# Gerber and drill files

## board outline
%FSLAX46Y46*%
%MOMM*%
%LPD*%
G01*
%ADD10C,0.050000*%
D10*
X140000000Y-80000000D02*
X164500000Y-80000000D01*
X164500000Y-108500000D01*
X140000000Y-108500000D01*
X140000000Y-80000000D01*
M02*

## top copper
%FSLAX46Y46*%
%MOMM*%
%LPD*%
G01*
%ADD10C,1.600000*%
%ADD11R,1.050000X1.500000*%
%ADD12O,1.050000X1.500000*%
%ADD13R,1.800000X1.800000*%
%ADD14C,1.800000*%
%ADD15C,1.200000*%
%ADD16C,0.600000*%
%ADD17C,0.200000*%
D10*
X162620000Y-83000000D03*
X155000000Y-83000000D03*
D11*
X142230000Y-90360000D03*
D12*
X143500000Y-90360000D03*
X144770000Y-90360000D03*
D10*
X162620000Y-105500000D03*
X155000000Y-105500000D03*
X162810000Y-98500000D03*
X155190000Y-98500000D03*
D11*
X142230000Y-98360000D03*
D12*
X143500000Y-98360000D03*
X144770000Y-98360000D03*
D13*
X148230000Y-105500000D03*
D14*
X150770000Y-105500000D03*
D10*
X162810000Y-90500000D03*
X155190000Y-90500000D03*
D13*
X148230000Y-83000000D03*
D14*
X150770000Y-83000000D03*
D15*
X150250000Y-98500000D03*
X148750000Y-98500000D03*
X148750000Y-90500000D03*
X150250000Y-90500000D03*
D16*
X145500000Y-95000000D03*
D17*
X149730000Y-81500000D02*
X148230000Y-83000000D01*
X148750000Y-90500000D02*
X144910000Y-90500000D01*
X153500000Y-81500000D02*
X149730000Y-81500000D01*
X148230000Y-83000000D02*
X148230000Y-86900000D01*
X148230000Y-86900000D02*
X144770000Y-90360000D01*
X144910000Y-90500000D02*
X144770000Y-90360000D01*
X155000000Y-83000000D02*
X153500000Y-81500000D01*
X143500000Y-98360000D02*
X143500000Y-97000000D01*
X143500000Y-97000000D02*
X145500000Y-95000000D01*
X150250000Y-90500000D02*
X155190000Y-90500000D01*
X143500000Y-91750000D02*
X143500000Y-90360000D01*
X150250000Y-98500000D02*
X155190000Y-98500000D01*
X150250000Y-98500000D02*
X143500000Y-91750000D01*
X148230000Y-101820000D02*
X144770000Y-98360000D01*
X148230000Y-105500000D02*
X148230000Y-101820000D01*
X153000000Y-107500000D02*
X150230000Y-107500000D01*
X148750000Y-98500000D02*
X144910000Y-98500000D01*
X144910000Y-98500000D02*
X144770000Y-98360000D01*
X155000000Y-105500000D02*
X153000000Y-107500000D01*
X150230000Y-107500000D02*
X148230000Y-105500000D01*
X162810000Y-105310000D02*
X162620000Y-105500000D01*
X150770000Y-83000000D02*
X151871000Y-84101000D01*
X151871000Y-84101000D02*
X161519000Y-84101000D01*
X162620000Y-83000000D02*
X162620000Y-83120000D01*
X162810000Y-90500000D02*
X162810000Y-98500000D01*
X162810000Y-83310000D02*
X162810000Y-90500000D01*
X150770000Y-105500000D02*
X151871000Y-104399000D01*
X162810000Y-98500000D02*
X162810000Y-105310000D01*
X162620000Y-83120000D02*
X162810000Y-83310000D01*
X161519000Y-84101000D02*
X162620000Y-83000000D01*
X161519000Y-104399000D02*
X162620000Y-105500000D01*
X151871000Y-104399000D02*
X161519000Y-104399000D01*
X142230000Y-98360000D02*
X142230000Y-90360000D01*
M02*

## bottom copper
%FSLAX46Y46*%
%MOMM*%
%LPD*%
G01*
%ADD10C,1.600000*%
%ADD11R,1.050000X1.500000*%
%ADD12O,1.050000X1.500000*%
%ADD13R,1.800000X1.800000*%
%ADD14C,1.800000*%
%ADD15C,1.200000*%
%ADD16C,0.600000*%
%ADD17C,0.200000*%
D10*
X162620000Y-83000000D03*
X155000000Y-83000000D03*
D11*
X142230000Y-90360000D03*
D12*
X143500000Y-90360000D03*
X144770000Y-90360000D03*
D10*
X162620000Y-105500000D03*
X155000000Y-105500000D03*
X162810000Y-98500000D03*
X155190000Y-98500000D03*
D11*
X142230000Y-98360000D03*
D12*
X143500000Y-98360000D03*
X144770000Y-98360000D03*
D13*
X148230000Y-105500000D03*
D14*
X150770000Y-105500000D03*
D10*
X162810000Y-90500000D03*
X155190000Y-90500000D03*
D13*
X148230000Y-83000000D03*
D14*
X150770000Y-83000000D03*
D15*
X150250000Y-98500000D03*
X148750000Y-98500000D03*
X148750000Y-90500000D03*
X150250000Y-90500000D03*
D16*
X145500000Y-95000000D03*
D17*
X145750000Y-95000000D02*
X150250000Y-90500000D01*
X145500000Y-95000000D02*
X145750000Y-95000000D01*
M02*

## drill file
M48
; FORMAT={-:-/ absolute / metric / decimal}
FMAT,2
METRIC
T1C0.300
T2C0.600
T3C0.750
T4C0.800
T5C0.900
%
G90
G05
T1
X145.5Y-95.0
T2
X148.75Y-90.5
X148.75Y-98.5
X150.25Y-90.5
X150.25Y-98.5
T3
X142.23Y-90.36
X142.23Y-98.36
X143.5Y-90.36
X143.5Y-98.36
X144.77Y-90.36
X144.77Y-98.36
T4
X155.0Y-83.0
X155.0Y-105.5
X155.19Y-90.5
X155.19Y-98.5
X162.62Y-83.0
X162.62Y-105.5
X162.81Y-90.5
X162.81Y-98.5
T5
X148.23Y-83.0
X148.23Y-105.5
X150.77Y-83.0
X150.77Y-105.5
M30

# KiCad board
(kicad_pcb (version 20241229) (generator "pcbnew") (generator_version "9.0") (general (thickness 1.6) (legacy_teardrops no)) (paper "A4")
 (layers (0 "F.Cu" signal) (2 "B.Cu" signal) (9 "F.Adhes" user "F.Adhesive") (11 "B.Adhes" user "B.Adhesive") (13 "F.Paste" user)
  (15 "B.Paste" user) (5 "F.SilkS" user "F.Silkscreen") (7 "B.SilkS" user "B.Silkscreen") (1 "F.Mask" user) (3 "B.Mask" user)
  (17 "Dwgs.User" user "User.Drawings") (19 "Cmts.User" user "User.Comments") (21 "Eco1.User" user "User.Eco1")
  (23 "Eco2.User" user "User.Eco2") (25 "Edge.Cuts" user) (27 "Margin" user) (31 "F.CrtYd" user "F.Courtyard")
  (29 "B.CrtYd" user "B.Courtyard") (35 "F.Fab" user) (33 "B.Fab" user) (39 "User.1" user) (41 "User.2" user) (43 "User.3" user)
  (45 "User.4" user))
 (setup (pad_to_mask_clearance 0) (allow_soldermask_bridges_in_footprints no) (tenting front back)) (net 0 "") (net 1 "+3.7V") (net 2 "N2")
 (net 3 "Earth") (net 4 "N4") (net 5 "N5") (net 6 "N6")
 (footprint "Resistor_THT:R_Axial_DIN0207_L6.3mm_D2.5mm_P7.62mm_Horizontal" (layer "F.Cu") (at 162.62 83 180)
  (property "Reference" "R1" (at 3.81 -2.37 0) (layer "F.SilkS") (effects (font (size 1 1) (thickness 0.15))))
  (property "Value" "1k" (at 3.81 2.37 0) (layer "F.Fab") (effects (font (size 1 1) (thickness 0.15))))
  (pad "1" thru_hole circle (at 0 0 180) (size 1.6 1.6) (drill 0.8) (layers "*.Cu" "*.Mask") (remove_unused_layers no) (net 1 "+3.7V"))
  (pad "2" thru_hole circle (at 7.62 0 180) (size 1.6 1.6) (drill 0.8) (layers "*.Cu" "*.Mask") (remove_unused_layers no) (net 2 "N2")))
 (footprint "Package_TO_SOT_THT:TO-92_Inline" (layer "F.Cu") (at 142.23 90.36)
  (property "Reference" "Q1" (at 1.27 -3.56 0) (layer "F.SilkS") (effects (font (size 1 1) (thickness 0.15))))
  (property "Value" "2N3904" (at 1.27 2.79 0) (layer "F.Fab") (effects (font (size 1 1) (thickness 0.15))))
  (pad "1" thru_hole rect (at 0 0) (size 1.05 1.5) (drill 0.75) (layers "*.Cu" "*.Mask") (remove_unused_layers no) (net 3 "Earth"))
  (pad "2" thru_hole oval (at 1.27 0) (size 1.05 1.5) (drill 0.75) (layers "*.Cu" "*.Mask") (remove_unused_layers no) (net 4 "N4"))
  (pad "3" thru_hole oval (at 2.54 0) (size 1.05 1.5) (drill 0.75) (layers "*.Cu" "*.Mask") (remove_unused_layers no) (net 2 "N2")))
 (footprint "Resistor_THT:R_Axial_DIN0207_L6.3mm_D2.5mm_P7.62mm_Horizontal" (layer "F.Cu") (at 162.62 105.5 180)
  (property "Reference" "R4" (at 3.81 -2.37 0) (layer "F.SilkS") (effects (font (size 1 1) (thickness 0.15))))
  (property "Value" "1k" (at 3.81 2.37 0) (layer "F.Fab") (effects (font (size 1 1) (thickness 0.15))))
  (pad "1" thru_hole circle (at 0 0 180) (size 1.6 1.6) (drill 0.8) (layers "*.Cu" "*.Mask") (remove_unused_layers no) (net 1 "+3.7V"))
  (pad "2" thru_hole circle (at 7.62 0 180) (size 1.6 1.6) (drill 0.8) (layers "*.Cu" "*.Mask") (remove_unused_layers no) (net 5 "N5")))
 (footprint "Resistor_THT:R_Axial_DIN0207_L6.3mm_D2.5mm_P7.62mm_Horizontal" (layer "F.Cu") (at 162.81 98.5 180)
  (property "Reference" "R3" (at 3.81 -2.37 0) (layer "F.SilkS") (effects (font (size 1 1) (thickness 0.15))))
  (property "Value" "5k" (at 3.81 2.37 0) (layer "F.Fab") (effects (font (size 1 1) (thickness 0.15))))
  (pad "1" thru_hole circle (at 0 0 180) (size 1.6 1.6) (drill 0.8) (layers "*.Cu" "*.Mask") (remove_unused_layers no) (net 1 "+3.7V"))
  (pad "2" thru_hole circle (at 7.62 0 180) (size 1.6 1.6) (drill 0.8) (layers "*.Cu" "*.Mask") (remove_unused_layers no) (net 4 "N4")))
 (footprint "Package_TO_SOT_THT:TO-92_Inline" (layer "F.Cu") (at 142.23 98.36)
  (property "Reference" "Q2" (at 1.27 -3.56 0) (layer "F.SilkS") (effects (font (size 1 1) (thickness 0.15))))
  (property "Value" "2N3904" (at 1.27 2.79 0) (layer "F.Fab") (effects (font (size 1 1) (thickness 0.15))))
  (pad "1" thru_hole rect (at 0 0) (size 1.05 1.5) (drill 0.75) (layers "*.Cu" "*.Mask") (remove_unused_layers no) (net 3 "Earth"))
  (pad "2" thru_hole oval (at 1.27 0) (size 1.05 1.5) (drill 0.75) (layers "*.Cu" "*.Mask") (remove_unused_layers no) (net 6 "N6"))
  (pad "3" thru_hole oval (at 2.54 0) (size 1.05 1.5) (drill 0.75) (layers "*.Cu" "*.Mask") (remove_unused_layers no) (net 5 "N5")))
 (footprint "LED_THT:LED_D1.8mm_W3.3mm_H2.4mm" (layer "F.Cu") (at 148.23 105.5)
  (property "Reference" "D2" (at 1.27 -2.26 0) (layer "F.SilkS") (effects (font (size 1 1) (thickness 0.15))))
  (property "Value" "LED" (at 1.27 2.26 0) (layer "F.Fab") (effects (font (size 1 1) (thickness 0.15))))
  (pad "1" thru_hole rect (at 0 0) (size 1.8 1.8) (drill 0.9) (layers "*.Cu" "*.Mask") (remove_unused_layers no) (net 5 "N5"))
  (pad "2" thru_hole circle (at 2.54 0) (size 1.8 1.8) (drill 0.9) (layers "*.Cu" "*.Mask") (remove_unused_layers no) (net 1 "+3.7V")))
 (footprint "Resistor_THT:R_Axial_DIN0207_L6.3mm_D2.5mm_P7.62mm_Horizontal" (layer "F.Cu") (at 162.81 90.5 180)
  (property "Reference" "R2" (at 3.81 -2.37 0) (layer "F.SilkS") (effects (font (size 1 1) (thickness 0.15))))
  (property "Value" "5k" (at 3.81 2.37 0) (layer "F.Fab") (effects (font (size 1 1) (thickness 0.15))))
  (pad "1" thru_hole circle (at 0 0 180) (size 1.6 1.6) (drill 0.8) (layers "*.Cu" "*.Mask") (remove_unused_layers no) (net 1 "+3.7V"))
  (pad "2" thru_hole circle (at 7.62 0 180) (size 1.6 1.6) (drill 0.8) (layers "*.Cu" "*.Mask") (remove_unused_layers no) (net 6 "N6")))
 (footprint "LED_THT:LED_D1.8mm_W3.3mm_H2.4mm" (layer "F.Cu") (at 148.23 83)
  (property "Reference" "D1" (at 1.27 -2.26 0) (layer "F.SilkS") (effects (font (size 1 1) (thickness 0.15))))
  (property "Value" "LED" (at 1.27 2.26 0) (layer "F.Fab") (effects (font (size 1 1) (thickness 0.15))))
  (pad "1" thru_hole rect (at 0 0) (size 1.8 1.8) (drill 0.9) (layers "*.Cu" "*.Mask") (remove_unused_layers no) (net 2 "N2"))
  (pad "2" thru_hole circle (at 2.54 0) (size 1.8 1.8) (drill 0.9) (layers "*.Cu" "*.Mask") (remove_unused_layers no) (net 1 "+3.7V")))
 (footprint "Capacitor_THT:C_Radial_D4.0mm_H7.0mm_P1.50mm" (layer "F.Cu") (at 150.25 98.5 180)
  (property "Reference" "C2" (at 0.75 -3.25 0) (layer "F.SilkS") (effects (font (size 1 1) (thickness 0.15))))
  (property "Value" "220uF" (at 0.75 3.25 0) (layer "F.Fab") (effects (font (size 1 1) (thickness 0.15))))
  (pad "1" thru_hole circle (at 0 0 180) (size 1.2 1.2) (drill 0.6) (layers "*.Cu" "*.Mask") (remove_unused_layers no) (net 4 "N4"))
  (pad "2" thru_hole circle (at 1.5 0 180) (size 1.2 1.2) (drill 0.6) (layers "*.Cu" "*.Mask") (remove_unused_layers no) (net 5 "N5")))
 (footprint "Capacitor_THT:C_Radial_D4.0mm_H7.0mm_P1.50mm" (layer "F.Cu") (at 148.75 90.5)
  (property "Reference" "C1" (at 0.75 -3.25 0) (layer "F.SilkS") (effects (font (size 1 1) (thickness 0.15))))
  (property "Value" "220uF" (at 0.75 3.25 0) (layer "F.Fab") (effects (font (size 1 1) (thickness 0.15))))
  (pad "1" thru_hole circle (at 0 0) (size 1.2 1.2) (drill 0.6) (layers "*.Cu" "*.Mask") (remove_unused_layers no) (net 2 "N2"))
  (pad "2" thru_hole circle (at 1.5 0) (size 1.2 1.2) (drill 0.6) (layers "*.Cu" "*.Mask") (remove_unused_layers no) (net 6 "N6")))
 (gr_rect (start 140 80) (end 164.5 108.5) (stroke (width 0.05) (type solid)) (fill no) (layer "Edge.Cuts"))
 (segment (start 149.73 81.5) (end 148.23 83) (width 0.2) (layer "F.Cu") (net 2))
 (segment (start 148.75 90.5) (end 144.91 90.5) (width 0.2) (layer "F.Cu") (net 2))
 (segment (start 153.5 81.5) (end 149.73 81.5) (width 0.2) (layer "F.Cu") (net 2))
 (segment (start 148.23 83) (end 148.23 86.9) (width 0.2) (layer "F.Cu") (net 2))
 (segment (start 148.23 86.9) (end 144.77 90.36) (width 0.2) (layer "F.Cu") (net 2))
 (segment (start 144.91 90.5) (end 144.77 90.36) (width 0.2) (layer "F.Cu") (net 2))
 (segment (start 155 83) (end 153.5 81.5) (width 0.2) (layer "F.Cu") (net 2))
 (segment (start 143.5 98.36) (end 143.5 97) (width 0.2) (layer "F.Cu") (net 6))
 (segment (start 143.5 97) (end 145.5 95) (width 0.2) (layer "F.Cu") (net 6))
 (segment (start 150.25 90.5) (end 155.19 90.5) (width 0.2) (layer "F.Cu") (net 6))
 (via (at 145.5 95) (size 0.6) (drill 0.3) (layers "F.Cu" "B.Cu") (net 6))
 (segment (start 145.75 95) (end 150.25 90.5) (width 0.2) (layer "B.Cu") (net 6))
 (segment (start 145.5 95) (end 145.75 95) (width 0.2) (layer "B.Cu") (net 6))
 (segment (start 143.5 91.75) (end 143.5 90.36) (width 0.2) (layer "F.Cu") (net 4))
 (segment (start 150.25 98.5) (end 155.19 98.5) (width 0.2) (layer "F.Cu") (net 4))
 (segment (start 150.25 98.5) (end 143.5 91.75) (width 0.2) (layer "F.Cu") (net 4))
 (segment (start 148.23 101.82) (end 144.77 98.36) (width 0.2) (layer "F.Cu") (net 5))
 (segment (start 148.23 105.5) (end 148.23 101.82) (width 0.2) (layer "F.Cu") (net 5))
 (segment (start 153 107.5) (end 150.23 107.5) (width 0.2) (layer "F.Cu") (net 5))
 (segment (start 148.75 98.5) (end 144.91 98.5) (width 0.2) (layer "F.Cu") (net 5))
 (segment (start 144.91 98.5) (end 144.77 98.36) (width 0.2) (layer "F.Cu") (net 5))
 (segment (start 155 105.5) (end 153 107.5) (width 0.2) (layer "F.Cu") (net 5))
 (segment (start 150.23 107.5) (end 148.23 105.5) (width 0.2) (layer "F.Cu") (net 5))
 (segment (start 162.81 105.31) (end 162.62 105.5) (width 0.2) (layer "F.Cu") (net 1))
 (segment (start 150.77 83) (end 151.871 84.101) (width 0.2) (layer "F.Cu") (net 1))
 (segment (start 151.871 84.101) (end 161.519 84.101) (width 0.2) (layer "F.Cu") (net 1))
 (segment (start 162.62 83) (end 162.62 83.12) (width 0.2) (layer "F.Cu") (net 1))
 (segment (start 162.81 90.5) (end 162.81 98.5) (width 0.2) (layer "F.Cu") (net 1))
 (segment (start 162.81 83.31) (end 162.81 90.5) (width 0.2) (layer "F.Cu") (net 1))
 (segment (start 150.77 105.5) (end 151.871 104.399) (width 0.2) (layer "F.Cu") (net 1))
 (segment (start 162.81 98.5) (end 162.81 105.31) (width 0.2) (layer "F.Cu") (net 1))
 (segment (start 162.62 83.12) (end 162.81 83.31) (width 0.2) (layer "F.Cu") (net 1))
 (segment (start 161.519 84.101) (end 162.62 83) (width 0.2) (layer "F.Cu") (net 1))
 (segment (start 161.519 104.399) (end 162.62 105.5) (width 0.2) (layer "F.Cu") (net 1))
 (segment (start 151.871 104.399) (end 161.519 104.399) (width 0.2) (layer "F.Cu") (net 1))
 (segment (start 142.23 98.36) (end 142.23 90.36) (width 0.2) (layer "F.Cu") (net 3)))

